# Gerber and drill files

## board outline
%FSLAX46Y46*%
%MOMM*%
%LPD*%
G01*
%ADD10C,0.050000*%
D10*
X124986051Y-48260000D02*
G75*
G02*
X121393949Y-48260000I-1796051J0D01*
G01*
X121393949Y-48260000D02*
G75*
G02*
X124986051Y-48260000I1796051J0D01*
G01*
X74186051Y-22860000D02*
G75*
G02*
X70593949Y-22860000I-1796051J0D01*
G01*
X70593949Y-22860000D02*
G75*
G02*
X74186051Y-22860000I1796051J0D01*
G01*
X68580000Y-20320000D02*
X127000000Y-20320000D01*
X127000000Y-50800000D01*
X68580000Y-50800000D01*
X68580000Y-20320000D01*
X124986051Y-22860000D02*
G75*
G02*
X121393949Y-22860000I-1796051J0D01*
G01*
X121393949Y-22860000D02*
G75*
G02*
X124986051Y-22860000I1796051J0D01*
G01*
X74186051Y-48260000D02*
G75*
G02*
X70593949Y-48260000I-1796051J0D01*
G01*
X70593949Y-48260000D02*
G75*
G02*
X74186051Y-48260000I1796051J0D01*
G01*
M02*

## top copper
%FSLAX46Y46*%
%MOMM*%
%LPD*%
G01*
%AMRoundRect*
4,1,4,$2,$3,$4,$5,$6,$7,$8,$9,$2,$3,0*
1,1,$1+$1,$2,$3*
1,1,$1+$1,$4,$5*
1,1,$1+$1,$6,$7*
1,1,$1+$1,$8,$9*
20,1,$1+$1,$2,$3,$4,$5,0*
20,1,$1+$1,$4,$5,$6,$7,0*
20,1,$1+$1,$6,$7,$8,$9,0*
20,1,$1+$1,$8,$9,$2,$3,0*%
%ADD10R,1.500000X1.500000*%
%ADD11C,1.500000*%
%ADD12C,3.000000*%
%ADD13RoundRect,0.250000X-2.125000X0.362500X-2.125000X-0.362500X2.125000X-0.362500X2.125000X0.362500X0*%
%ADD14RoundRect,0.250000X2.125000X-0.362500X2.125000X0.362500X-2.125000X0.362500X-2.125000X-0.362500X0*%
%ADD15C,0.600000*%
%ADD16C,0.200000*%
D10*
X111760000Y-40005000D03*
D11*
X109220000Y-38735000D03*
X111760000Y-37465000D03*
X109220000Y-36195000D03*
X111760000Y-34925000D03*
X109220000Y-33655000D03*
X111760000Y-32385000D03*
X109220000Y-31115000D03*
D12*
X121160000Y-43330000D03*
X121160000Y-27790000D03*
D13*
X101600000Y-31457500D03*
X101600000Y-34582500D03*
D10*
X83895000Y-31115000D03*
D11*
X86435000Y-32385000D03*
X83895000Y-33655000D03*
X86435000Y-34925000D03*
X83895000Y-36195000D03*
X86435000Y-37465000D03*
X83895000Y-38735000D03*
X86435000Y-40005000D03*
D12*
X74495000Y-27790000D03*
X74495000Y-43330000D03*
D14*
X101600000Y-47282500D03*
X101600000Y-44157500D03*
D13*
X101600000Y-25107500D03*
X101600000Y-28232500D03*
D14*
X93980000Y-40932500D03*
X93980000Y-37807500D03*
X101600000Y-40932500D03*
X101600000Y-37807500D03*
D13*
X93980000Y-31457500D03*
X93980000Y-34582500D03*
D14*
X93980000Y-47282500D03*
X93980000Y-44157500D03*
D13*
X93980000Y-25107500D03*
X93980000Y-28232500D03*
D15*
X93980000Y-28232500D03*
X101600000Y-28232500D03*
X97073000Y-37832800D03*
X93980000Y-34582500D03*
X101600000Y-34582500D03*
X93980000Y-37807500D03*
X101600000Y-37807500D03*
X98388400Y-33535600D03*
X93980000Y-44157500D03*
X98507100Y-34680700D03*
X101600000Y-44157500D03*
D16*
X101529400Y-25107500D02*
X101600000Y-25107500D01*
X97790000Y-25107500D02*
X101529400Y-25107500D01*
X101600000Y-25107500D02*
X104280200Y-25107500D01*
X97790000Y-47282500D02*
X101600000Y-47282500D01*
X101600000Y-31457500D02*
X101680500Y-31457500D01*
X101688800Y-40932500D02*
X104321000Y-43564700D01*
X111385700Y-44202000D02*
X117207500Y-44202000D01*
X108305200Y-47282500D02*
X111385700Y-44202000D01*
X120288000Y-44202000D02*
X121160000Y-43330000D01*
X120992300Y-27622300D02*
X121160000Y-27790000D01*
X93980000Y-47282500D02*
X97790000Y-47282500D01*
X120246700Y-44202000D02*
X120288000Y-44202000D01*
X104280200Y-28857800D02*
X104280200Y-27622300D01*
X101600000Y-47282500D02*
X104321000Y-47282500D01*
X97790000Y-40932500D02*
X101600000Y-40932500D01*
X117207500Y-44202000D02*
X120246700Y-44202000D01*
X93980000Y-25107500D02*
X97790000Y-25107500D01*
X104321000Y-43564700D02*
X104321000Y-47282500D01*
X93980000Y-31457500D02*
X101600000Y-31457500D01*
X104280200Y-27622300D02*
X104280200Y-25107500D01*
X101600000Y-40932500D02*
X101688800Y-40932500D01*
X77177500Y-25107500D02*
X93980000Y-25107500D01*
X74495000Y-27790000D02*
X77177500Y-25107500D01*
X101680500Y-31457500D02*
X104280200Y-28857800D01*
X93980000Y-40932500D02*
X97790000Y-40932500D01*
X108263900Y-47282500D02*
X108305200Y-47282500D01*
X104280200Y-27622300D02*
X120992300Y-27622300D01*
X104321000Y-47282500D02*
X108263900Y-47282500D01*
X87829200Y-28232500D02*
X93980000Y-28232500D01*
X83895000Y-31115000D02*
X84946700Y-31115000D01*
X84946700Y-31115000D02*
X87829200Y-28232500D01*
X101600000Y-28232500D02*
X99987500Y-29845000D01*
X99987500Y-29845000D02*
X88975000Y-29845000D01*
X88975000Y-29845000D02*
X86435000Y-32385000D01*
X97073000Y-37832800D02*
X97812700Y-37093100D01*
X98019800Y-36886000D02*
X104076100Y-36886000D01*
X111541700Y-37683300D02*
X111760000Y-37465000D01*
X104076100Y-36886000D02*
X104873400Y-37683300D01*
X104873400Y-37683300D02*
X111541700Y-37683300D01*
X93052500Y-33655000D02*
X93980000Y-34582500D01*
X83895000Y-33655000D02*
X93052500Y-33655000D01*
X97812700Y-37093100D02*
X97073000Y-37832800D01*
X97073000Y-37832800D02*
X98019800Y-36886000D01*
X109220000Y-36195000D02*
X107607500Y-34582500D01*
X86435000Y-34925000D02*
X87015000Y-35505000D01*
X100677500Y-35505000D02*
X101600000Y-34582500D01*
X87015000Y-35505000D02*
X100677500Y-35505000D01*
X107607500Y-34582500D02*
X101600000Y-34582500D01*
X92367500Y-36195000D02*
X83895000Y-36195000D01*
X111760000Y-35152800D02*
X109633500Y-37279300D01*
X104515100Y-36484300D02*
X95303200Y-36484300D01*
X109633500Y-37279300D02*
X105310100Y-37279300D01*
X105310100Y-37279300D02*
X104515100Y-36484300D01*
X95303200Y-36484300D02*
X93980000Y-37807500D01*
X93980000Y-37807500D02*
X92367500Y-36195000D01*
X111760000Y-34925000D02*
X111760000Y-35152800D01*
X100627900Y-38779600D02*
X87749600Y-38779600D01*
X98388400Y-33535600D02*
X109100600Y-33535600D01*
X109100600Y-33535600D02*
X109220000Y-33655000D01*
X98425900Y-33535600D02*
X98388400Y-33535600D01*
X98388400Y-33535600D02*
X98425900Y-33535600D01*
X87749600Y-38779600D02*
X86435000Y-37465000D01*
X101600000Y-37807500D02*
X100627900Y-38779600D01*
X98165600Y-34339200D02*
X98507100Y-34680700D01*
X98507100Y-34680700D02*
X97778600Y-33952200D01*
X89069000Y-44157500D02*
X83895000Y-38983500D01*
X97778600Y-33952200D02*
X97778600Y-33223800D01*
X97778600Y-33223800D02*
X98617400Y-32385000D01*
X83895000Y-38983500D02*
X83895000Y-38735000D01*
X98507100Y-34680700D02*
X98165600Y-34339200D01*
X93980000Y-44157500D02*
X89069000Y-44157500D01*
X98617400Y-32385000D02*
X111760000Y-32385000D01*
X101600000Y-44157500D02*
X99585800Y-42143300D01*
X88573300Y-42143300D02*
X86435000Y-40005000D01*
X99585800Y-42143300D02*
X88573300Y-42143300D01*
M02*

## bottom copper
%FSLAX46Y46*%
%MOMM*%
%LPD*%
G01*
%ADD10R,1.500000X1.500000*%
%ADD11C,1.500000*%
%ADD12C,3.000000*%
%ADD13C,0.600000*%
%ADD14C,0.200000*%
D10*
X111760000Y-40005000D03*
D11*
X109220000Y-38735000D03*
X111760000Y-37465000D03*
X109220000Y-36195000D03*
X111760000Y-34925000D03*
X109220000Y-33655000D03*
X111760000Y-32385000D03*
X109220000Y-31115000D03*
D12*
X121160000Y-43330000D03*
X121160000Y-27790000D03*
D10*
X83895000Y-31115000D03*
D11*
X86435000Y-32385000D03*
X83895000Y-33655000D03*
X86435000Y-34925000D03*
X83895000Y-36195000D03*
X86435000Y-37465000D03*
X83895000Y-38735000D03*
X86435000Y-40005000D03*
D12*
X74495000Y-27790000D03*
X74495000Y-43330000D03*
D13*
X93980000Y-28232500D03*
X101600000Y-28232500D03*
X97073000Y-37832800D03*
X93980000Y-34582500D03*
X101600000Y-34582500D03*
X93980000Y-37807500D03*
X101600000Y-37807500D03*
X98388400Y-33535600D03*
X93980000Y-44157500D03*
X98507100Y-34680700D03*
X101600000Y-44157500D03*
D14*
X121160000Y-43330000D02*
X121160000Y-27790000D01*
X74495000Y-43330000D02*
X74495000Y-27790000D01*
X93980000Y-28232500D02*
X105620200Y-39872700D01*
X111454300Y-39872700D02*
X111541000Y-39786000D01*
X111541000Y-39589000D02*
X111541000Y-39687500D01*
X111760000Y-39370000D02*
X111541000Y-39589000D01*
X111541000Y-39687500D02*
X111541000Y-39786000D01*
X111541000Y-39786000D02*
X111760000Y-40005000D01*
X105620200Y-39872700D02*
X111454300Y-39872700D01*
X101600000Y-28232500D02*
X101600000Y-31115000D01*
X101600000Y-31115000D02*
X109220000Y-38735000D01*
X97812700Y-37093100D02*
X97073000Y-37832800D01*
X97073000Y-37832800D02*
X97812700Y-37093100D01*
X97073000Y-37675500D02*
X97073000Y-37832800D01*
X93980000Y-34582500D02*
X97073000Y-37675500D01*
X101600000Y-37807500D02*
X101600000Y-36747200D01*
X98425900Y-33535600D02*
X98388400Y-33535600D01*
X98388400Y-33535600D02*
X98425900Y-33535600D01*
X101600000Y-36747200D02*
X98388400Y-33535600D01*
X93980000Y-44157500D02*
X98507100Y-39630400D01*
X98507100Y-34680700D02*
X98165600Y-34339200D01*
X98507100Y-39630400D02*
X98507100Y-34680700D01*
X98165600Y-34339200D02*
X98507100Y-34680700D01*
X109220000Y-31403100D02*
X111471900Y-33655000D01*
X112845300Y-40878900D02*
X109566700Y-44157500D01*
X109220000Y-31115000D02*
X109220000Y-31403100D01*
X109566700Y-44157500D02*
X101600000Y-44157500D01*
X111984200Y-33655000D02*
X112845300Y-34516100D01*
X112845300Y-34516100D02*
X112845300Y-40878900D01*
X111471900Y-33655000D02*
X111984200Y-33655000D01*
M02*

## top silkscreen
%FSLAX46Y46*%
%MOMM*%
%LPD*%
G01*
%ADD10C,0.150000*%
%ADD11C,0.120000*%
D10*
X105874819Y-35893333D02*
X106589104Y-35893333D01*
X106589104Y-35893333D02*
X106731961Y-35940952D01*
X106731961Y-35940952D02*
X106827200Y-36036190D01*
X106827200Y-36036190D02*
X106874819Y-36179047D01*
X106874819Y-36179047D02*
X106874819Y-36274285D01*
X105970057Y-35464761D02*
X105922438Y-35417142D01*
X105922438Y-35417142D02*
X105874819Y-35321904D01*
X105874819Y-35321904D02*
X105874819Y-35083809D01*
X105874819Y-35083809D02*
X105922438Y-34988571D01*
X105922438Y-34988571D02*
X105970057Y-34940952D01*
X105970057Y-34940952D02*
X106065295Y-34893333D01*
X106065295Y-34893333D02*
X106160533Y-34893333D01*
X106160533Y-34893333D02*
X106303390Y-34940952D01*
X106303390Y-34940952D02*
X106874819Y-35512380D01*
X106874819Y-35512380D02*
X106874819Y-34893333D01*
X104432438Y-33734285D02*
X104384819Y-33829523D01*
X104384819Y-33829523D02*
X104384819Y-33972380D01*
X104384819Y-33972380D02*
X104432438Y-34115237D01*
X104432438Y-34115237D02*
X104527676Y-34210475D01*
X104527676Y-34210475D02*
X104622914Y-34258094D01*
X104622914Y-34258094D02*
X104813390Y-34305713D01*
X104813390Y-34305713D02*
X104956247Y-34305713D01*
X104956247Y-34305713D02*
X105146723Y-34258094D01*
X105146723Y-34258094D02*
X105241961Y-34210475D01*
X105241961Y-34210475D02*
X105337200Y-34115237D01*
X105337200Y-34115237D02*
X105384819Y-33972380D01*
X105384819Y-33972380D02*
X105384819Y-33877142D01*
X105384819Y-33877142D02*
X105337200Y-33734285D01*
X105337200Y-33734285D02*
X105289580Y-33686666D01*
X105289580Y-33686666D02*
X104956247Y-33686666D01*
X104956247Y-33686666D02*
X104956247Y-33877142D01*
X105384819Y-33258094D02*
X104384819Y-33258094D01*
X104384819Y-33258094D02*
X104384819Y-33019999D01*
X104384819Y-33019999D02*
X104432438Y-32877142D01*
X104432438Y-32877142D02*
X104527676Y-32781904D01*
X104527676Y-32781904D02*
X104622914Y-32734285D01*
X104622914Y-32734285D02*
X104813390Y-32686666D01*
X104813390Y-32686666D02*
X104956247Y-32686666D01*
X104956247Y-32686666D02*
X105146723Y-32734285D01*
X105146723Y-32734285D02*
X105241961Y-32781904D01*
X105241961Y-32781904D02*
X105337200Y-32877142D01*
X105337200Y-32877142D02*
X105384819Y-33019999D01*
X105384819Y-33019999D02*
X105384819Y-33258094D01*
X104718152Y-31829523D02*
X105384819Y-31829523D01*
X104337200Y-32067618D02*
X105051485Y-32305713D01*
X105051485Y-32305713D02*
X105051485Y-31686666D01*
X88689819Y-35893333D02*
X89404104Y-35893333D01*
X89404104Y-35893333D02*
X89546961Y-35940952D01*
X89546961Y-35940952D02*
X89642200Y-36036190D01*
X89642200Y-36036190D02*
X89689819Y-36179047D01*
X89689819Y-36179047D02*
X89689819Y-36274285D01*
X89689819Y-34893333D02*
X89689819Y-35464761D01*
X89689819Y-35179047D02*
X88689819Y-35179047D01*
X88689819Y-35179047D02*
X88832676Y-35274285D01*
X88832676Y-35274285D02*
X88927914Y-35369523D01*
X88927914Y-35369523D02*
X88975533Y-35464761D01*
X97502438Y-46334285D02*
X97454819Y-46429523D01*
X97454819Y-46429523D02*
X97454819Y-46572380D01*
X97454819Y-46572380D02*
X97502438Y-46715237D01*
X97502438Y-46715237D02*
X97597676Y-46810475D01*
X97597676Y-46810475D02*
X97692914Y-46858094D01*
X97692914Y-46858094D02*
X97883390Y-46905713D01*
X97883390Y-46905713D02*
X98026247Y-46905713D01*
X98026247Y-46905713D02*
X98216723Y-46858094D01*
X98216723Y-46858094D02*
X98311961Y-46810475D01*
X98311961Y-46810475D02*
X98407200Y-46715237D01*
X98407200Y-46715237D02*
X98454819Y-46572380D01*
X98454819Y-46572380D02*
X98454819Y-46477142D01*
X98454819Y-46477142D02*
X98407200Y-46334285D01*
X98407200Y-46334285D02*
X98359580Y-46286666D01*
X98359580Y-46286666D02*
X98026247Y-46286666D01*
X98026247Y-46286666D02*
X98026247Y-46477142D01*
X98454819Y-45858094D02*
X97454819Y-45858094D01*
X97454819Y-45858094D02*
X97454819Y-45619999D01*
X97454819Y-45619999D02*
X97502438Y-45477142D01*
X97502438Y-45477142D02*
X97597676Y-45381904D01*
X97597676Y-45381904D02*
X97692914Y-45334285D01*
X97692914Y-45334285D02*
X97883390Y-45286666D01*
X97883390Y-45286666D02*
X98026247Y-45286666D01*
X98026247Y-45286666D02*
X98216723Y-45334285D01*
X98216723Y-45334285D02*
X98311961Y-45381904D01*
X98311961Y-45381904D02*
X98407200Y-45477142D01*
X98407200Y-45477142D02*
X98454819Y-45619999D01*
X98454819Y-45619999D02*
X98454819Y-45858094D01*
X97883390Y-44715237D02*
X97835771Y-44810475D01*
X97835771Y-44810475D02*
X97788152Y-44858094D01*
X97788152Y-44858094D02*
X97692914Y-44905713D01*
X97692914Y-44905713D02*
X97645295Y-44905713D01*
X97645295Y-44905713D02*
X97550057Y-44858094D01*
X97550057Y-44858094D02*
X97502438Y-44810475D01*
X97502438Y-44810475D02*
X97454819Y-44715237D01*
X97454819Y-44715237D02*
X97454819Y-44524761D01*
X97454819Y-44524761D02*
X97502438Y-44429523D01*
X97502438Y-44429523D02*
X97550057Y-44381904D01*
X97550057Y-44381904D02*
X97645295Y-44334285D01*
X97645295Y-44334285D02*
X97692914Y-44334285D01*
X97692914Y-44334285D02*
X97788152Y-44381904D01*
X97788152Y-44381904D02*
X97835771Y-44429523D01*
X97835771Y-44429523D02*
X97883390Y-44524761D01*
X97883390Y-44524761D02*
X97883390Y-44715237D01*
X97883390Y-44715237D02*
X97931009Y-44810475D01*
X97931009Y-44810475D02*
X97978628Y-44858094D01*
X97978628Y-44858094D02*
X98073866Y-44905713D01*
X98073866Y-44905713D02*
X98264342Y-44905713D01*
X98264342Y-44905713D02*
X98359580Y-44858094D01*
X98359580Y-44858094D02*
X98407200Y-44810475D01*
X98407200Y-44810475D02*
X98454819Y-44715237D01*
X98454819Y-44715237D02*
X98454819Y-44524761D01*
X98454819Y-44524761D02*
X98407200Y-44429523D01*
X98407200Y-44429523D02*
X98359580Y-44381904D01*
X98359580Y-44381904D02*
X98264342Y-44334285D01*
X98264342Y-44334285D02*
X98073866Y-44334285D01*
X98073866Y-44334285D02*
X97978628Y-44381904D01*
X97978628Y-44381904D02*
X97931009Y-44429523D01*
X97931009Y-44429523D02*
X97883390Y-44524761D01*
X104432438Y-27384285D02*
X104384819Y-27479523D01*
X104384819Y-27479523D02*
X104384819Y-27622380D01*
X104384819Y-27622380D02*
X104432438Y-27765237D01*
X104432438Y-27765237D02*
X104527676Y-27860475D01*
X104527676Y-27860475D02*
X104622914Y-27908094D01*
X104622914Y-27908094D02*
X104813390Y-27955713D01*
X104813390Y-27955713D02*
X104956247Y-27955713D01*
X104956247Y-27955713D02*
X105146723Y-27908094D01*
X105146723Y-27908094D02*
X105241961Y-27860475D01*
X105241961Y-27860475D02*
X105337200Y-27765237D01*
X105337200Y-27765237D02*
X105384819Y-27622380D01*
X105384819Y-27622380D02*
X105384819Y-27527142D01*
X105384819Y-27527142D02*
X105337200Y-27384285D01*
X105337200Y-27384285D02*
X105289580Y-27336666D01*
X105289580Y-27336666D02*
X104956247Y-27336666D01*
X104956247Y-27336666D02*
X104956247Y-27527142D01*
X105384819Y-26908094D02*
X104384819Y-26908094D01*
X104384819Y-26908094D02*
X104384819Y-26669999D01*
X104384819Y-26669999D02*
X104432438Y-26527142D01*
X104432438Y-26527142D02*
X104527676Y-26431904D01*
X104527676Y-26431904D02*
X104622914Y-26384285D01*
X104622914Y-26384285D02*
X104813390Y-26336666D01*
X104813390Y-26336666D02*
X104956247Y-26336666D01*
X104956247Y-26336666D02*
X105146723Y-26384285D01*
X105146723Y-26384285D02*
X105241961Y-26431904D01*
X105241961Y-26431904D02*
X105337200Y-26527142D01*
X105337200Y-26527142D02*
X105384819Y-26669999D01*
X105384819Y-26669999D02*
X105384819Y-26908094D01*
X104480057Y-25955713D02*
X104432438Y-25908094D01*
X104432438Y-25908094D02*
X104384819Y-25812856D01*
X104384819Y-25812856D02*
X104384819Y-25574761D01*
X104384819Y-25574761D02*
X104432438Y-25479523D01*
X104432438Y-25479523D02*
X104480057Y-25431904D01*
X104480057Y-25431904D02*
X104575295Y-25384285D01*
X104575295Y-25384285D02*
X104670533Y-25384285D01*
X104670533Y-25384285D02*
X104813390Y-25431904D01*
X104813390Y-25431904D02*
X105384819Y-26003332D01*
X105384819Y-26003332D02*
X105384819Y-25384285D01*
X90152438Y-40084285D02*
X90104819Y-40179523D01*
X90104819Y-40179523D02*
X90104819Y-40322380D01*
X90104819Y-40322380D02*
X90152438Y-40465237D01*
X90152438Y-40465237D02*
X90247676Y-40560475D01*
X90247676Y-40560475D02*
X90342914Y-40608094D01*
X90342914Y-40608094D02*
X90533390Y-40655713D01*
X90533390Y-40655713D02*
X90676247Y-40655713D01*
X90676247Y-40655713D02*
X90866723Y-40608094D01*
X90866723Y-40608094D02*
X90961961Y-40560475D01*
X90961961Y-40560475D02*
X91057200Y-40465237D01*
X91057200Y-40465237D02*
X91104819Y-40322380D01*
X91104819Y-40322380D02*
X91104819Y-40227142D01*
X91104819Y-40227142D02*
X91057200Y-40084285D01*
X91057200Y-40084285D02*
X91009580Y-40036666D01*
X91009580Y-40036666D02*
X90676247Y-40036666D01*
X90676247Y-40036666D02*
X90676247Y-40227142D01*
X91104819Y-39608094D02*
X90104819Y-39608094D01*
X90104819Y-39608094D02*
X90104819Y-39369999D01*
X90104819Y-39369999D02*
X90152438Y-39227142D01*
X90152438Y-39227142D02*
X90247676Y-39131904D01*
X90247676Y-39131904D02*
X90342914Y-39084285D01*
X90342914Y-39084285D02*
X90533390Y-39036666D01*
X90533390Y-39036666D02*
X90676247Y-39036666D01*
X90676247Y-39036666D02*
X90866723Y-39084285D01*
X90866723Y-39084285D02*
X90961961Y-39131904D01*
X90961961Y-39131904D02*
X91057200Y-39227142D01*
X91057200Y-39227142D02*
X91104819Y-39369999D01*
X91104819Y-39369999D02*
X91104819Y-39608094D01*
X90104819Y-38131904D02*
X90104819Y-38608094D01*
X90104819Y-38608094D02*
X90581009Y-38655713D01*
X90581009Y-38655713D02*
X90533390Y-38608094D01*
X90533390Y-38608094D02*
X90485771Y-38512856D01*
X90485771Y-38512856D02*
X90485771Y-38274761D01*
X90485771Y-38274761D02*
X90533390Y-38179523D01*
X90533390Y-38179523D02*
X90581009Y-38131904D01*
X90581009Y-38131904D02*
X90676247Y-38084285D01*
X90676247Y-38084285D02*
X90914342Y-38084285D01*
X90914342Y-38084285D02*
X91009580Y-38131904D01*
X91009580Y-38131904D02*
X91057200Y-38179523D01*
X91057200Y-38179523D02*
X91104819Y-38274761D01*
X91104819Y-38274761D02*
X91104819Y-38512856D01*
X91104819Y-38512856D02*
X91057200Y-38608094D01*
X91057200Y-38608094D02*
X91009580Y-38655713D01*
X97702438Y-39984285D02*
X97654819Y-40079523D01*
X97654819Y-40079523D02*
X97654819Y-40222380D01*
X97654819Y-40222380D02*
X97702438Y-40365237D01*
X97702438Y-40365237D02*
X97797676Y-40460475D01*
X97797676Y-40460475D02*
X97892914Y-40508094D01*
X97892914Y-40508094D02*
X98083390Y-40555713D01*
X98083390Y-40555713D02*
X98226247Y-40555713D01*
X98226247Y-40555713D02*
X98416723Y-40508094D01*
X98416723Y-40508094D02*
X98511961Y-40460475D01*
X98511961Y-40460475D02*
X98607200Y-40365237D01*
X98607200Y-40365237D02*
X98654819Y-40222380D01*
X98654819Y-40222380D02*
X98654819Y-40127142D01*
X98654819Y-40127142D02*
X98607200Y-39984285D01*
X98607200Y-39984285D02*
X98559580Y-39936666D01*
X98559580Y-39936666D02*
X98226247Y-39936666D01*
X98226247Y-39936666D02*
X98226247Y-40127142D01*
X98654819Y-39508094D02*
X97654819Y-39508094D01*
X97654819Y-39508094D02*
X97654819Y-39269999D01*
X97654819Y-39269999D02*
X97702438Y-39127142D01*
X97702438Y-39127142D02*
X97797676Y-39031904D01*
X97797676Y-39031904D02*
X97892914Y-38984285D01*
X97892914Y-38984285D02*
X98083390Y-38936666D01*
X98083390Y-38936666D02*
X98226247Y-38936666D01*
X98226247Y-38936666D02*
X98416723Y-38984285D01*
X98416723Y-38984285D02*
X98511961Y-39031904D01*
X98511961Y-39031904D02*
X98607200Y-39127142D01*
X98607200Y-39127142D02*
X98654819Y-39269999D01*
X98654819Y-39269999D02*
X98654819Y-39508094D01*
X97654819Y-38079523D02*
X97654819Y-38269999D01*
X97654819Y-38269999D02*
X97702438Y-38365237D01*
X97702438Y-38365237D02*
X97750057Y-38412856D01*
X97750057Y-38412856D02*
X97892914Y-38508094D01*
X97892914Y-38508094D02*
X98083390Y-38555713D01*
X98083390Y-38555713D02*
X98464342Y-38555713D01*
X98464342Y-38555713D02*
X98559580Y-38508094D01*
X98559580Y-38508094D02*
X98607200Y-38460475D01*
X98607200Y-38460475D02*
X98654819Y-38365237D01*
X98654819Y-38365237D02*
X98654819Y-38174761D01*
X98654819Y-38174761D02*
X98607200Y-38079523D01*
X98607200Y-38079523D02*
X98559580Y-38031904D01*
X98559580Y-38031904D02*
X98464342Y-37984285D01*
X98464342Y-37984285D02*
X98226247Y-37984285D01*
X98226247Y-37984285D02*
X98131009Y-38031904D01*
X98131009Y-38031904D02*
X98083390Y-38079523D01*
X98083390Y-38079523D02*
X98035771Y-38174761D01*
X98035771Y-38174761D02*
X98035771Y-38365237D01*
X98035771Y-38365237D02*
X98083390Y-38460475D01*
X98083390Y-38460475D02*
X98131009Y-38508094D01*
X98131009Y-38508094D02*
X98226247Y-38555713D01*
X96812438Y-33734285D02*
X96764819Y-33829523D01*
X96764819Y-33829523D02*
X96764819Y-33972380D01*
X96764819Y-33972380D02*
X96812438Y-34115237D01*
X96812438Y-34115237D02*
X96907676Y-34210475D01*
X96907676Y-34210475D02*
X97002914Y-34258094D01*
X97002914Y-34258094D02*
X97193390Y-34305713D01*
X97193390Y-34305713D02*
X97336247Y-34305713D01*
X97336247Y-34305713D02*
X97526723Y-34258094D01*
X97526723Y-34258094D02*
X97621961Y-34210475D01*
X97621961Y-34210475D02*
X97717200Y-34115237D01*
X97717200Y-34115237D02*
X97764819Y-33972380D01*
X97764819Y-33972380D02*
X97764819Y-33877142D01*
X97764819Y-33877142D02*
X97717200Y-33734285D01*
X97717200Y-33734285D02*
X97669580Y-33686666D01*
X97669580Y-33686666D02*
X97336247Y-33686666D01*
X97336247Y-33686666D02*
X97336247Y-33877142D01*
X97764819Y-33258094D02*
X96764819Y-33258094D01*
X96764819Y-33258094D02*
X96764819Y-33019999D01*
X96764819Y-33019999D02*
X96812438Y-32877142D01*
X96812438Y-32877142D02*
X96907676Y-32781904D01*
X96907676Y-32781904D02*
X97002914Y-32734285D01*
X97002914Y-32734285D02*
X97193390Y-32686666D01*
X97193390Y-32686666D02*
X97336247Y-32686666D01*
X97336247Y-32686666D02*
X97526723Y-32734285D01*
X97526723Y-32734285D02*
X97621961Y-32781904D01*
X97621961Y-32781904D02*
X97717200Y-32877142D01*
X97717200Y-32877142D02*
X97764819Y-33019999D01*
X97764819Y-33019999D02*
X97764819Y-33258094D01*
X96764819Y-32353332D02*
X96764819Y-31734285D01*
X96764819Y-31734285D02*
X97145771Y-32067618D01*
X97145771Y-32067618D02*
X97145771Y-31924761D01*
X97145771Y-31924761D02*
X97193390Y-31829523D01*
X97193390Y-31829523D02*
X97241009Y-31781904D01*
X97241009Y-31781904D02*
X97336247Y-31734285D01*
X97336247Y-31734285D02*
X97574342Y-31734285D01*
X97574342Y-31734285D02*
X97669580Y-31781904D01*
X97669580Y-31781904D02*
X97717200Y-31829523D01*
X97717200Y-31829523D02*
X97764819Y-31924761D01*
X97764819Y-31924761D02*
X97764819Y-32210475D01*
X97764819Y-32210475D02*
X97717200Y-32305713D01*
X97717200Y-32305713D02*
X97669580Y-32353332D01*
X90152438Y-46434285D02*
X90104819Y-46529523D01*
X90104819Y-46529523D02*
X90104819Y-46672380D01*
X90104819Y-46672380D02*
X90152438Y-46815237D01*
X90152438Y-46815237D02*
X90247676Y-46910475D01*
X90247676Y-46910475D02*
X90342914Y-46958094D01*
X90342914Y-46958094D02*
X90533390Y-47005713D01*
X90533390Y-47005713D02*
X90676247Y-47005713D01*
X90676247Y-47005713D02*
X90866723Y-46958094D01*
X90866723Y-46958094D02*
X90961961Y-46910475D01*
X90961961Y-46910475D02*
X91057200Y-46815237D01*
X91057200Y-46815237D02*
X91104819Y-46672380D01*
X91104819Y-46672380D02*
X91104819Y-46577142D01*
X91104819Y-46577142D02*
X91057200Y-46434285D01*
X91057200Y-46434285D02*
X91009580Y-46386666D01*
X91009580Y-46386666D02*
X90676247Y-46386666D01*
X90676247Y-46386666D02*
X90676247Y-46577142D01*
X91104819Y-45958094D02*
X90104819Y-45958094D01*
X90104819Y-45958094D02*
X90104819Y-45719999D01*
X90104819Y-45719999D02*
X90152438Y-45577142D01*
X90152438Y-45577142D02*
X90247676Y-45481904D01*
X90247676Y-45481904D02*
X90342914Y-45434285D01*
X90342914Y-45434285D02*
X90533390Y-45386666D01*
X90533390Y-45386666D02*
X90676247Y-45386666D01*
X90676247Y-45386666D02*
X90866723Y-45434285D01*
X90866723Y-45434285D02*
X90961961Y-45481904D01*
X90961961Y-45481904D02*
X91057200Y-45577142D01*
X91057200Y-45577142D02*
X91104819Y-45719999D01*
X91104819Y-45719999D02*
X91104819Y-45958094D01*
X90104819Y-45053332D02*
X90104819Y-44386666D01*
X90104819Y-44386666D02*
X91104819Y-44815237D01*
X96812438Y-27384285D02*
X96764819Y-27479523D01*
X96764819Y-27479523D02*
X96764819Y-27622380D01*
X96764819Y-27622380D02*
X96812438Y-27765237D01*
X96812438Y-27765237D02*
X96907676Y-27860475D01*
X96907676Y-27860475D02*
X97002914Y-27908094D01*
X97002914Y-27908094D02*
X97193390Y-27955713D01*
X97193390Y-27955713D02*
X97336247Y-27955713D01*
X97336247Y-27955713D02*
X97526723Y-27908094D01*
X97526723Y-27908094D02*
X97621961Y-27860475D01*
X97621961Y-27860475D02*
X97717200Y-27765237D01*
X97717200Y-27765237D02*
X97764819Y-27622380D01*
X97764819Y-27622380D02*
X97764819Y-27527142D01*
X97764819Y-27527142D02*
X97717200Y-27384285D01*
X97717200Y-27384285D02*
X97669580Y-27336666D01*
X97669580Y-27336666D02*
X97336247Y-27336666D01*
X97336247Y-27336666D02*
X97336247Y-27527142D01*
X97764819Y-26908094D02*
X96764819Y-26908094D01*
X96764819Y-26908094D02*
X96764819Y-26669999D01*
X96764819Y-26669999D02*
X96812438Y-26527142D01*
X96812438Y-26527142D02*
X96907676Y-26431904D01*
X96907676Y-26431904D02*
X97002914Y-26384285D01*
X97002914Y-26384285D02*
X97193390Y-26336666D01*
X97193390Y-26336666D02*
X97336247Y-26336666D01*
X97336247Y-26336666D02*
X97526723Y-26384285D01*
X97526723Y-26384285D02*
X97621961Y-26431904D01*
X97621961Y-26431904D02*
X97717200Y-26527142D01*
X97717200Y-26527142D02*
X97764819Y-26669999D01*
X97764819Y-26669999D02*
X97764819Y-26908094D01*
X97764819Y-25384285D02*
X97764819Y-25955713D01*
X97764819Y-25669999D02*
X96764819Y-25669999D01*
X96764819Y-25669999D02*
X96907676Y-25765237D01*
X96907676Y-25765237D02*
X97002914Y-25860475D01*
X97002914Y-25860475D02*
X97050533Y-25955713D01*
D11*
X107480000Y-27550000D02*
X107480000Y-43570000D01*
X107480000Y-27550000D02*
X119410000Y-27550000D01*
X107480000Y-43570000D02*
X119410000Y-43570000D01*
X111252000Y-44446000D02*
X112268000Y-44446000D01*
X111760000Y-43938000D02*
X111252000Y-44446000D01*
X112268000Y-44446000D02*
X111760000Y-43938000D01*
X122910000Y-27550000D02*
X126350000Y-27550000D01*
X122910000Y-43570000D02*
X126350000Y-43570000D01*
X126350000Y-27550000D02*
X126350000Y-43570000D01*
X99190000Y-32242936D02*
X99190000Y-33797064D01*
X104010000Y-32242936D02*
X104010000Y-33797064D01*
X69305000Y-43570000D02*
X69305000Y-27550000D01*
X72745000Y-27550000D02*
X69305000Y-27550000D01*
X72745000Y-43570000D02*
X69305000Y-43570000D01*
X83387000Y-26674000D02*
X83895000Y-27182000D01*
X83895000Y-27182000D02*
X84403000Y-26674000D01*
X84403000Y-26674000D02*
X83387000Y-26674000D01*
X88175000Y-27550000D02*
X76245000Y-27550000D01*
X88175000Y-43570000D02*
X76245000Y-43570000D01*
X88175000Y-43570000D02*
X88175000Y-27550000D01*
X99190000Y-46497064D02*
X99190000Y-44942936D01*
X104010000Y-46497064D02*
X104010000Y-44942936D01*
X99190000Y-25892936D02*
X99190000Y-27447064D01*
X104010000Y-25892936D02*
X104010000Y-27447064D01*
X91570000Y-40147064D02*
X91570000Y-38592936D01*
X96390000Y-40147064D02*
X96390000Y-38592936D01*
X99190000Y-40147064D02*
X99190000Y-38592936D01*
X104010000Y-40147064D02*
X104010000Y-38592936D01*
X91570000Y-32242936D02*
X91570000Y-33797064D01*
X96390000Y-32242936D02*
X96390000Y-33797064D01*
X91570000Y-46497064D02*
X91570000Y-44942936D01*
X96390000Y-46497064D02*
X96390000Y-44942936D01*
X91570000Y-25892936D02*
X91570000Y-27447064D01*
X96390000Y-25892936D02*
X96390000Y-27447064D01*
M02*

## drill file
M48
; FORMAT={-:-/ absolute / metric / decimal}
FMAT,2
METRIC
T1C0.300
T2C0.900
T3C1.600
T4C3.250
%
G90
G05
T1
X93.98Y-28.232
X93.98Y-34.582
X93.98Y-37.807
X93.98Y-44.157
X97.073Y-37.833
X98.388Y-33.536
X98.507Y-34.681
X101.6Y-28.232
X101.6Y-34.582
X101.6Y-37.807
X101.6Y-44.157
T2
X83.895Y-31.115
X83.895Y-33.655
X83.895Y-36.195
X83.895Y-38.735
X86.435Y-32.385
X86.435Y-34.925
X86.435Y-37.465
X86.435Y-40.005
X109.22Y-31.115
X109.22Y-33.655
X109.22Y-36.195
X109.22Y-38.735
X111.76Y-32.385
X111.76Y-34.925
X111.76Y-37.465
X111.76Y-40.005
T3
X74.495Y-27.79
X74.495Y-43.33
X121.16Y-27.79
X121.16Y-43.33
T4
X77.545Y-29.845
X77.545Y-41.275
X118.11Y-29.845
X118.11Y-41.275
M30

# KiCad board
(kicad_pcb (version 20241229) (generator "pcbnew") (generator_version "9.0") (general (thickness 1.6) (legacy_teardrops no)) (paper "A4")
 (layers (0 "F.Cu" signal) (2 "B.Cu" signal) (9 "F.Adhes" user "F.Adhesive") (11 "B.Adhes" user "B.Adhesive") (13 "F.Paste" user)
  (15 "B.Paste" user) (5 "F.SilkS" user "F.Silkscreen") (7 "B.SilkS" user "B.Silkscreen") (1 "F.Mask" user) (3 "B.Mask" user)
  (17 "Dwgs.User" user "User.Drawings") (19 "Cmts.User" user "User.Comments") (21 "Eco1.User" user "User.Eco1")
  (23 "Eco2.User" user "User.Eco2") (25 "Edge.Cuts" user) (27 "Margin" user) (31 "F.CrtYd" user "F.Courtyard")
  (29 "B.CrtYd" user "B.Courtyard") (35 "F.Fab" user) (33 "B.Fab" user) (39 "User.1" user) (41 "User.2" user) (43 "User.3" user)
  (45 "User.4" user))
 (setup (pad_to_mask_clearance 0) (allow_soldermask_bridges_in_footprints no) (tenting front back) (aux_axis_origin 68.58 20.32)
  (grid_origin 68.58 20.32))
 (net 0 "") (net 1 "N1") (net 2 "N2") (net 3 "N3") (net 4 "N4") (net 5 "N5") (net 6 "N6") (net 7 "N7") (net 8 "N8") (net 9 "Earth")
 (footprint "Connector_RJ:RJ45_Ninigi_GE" (layer "F.Cu") (at 111.76 40.005 90)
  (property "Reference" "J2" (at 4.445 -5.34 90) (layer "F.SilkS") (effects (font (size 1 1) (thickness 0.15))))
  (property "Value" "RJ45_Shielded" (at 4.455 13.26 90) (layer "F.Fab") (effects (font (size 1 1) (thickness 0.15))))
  (fp_line (start 12.455 -4.28) (end -3.565 -4.28) (stroke (width 0.12) (type solid)) (layer "F.SilkS"))
  (fp_line (start 12.455 -4.28) (end 12.455 7.65) (stroke (width 0.12) (type solid)) (layer "F.SilkS"))
  (fp_line (start -3.565 -4.28) (end -3.565 7.65) (stroke (width 0.12) (type solid)) (layer "F.SilkS"))
  (fp_line (start -4.441 -0.508) (end -4.441 0.508) (stroke (width 0.12) (type solid)) (layer "F.SilkS"))
  (fp_line (start -3.933 0) (end -4.441 -0.508) (stroke (width 0.12) (type solid)) (layer "F.SilkS"))
  (fp_line (start -4.441 0.508) (end -3.933 0) (stroke (width 0.12) (type solid)) (layer "F.SilkS"))
  (fp_line (start 12.455 11.15) (end 12.455 14.59) (stroke (width 0.12) (type solid)) (layer "F.SilkS"))
  (fp_line (start -3.565 11.15) (end -3.565 14.59) (stroke (width 0.12) (type solid)) (layer "F.SilkS"))
  (fp_line (start 12.455 14.59) (end -3.565 14.59) (stroke (width 0.12) (type solid)) (layer "F.SilkS"))
  (pad "" np_thru_hole circle (at -1.27 6.35 90) (size 3.25 3.25) (drill 3.25) (layers "*.Cu" "*.Mask"))
  (pad "" np_thru_hole circle (at 10.16 6.35 270) (size 3.25 3.25) (drill 3.25) (layers "*.Cu" "*.Mask"))
  (pad "1" thru_hole rect (at 0 0 270) (size 1.5 1.5) (drill 0.9) (layers "*.Cu" "*.Mask") (remove_unused_layers no) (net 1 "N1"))
  (pad "2" thru_hole circle (at 1.27 -2.54 270) (size 1.5 1.5) (drill 0.9) (layers "*.Cu" "*.Mask") (remove_unused_layers no) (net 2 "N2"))
  (pad "3" thru_hole circle (at 2.54 0 270) (size 1.5 1.5) (drill 0.9) (layers "*.Cu" "*.Mask") (remove_unused_layers no) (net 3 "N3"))
  (pad "4" thru_hole circle (at 3.81 -2.54 270) (size 1.5 1.5) (drill 0.9) (layers "*.Cu" "*.Mask") (remove_unused_layers no) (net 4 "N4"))
  (pad "5" thru_hole circle (at 5.08 0 270) (size 1.5 1.5) (drill 0.9) (layers "*.Cu" "*.Mask") (remove_unused_layers no) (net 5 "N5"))
  (pad "6" thru_hole circle (at 6.35 -2.54 270) (size 1.5 1.5) (drill 0.9) (layers "*.Cu" "*.Mask") (remove_unused_layers no) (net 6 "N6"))
  (pad "7" thru_hole circle (at 7.62 0 270) (size 1.5 1.5) (drill 0.9) (layers "*.Cu" "*.Mask") (remove_unused_layers no) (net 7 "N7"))
  (pad "8" thru_hole circle (at 8.89 -2.54 270) (size 1.5 1.5) (drill 0.9) (layers "*.Cu" "*.Mask") (remove_unused_layers no) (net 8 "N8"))
  (pad "SH" thru_hole circle (at -3.325 9.4 90) (size 3 3) (drill 1.6) (layers "*.Cu" "*.Mask") (remove_unused_layers no) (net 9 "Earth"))
  (pad "SH" thru_hole circle (at 12.215 9.4 270) (size 3 3) (drill 1.6) (layers "*.Cu" "*.Mask") (remove_unused_layers no) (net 9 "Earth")))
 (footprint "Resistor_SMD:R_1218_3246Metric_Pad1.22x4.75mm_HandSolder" (layer "F.Cu") (at 101.6 33.02 -90)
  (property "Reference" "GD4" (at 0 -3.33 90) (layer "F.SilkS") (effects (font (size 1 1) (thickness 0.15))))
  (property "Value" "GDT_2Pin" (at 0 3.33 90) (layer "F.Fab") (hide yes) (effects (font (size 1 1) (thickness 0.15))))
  (fp_line (start -0.777064 2.41) (end 0.777064 2.41) (stroke (width 0.12) (type solid)) (layer "F.SilkS"))
  (fp_line (start -0.777064 -2.41) (end 0.777064 -2.41) (stroke (width 0.12) (type solid)) (layer "F.SilkS"))
  (pad "1" smd roundrect (at -1.5625 0 270) (size 1.225 4.75) (layers "F.Cu" "F.Mask" "F.Paste") (roundrect_rratio 0.204082) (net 9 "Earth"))
  (pad "2" smd roundrect (at 1.5625 0 270) (size 1.225 4.75) (layers "F.Cu" "F.Mask" "F.Paste") (roundrect_rratio 0.204082) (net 4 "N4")))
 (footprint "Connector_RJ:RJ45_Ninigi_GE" (layer "F.Cu") (at 83.895 31.115 -90)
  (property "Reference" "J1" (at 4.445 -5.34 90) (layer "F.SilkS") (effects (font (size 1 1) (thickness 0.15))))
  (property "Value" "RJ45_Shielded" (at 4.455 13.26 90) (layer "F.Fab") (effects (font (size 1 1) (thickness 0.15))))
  (fp_line (start 12.455 14.59) (end -3.565 14.59) (stroke (width 0.12) (type solid)) (layer "F.SilkS"))
  (fp_line (start -3.565 11.15) (end -3.565 14.59) (stroke (width 0.12) (type solid)) (layer "F.SilkS"))
  (fp_line (start 12.455 11.15) (end 12.455 14.59) (stroke (width 0.12) (type solid)) (layer "F.SilkS"))
  (fp_line (start -4.441 0.508) (end -3.933 0) (stroke (width 0.12) (type solid)) (layer "F.SilkS"))
  (fp_line (start -3.933 0) (end -4.441 -0.508) (stroke (width 0.12) (type solid)) (layer "F.SilkS"))
  (fp_line (start -4.441 -0.508) (end -4.441 0.508) (stroke (width 0.12) (type solid)) (layer "F.SilkS"))
  (fp_line (start -3.565 -4.28) (end -3.565 7.65) (stroke (width 0.12) (type solid)) (layer "F.SilkS"))
  (fp_line (start 12.455 -4.28) (end 12.455 7.65) (stroke (width 0.12) (type solid)) (layer "F.SilkS"))
  (fp_line (start 12.455 -4.28) (end -3.565 -4.28) (stroke (width 0.12) (type solid)) (layer "F.SilkS"))
  (pad "" np_thru_hole circle (at -1.27 6.35 270) (size 3.25 3.25) (drill 3.25) (layers "*.Cu" "*.Mask"))
  (pad "" np_thru_hole circle (at 10.16 6.35 90) (size 3.25 3.25) (drill 3.25) (layers "*.Cu" "*.Mask"))
  (pad "1" thru_hole rect (at 0 0 90) (size 1.5 1.5) (drill 0.9) (layers "*.Cu" "*.Mask") (remove_unused_layers no) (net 1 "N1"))
  (pad "2" thru_hole circle (at 1.27 -2.54 90) (size 1.5 1.5) (drill 0.9) (layers "*.Cu" "*.Mask") (remove_unused_layers no) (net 2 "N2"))
  (pad "3" thru_hole circle (at 2.54 0 90) (size 1.5 1.5) (drill 0.9) (layers "*.Cu" "*.Mask") (remove_unused_layers no) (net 3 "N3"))
  (pad "4" thru_hole circle (at 3.81 -2.54 90) (size 1.5 1.5) (drill 0.9) (layers "*.Cu" "*.Mask") (remove_unused_layers no) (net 4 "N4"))
  (pad "5" thru_hole circle (at 5.08 0 90) (size 1.5 1.5) (drill 0.9) (layers "*.Cu" "*.Mask") (remove_unused_layers no) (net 5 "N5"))
  (pad "6" thru_hole circle (at 6.35 -2.54 90) (size 1.5 1.5) (drill 0.9) (layers "*.Cu" "*.Mask") (remove_unused_layers no) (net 6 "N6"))
  (pad "7" thru_hole circle (at 7.62 0 90) (size 1.5 1.5) (drill 0.9) (layers "*.Cu" "*.Mask") (remove_unused_layers no) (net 7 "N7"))
  (pad "8" thru_hole circle (at 8.89 -2.54 90) (size 1.5 1.5) (drill 0.9) (layers "*.Cu" "*.Mask") (remove_unused_layers no) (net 8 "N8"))
  (pad "SH" thru_hole circle (at -3.325 9.4 270) (size 3 3) (drill 1.6) (layers "*.Cu" "*.Mask") (remove_unused_layers no) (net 9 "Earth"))
  (pad "SH" thru_hole circle (at 12.215 9.4 90) (size 3 3) (drill 1.6) (layers "*.Cu" "*.Mask") (remove_unused_layers no) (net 9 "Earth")))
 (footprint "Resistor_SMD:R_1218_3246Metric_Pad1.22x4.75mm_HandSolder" (layer "F.Cu") (at 101.6 45.72 90)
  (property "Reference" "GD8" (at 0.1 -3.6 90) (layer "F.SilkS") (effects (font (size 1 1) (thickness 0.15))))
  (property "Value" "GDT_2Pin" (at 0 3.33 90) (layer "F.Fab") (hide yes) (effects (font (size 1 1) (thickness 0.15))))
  (fp_line (start -0.777064 -2.41) (end 0.777064 -2.41) (stroke (width 0.12) (type solid)) (layer "F.SilkS"))
  (fp_line (start -0.777064 2.41) (end 0.777064 2.41) (stroke (width 0.12) (type solid)) (layer "F.SilkS"))
  (pad "1" smd roundrect (at -1.5625 0 90) (size 1.225 4.75) (layers "F.Cu" "F.Mask" "F.Paste") (roundrect_rratio 0.204082) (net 9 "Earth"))
  (pad "2" smd roundrect (at 1.5625 0 90) (size 1.225 4.75) (layers "F.Cu" "F.Mask" "F.Paste") (roundrect_rratio 0.204082) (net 8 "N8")))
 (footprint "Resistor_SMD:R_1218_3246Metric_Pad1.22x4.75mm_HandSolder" (layer "F.Cu") (at 101.6 26.67 -90)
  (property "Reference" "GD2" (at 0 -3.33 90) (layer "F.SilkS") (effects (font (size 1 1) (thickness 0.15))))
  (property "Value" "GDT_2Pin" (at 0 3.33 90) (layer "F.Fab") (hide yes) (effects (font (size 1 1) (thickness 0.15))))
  (fp_line (start -0.777064 2.41) (end 0.777064 2.41) (stroke (width 0.12) (type solid)) (layer "F.SilkS"))
  (fp_line (start -0.777064 -2.41) (end 0.777064 -2.41) (stroke (width 0.12) (type solid)) (layer "F.SilkS"))
  (pad "1" smd roundrect (at -1.5625 0 270) (size 1.225 4.75) (layers "F.Cu" "F.Mask" "F.Paste") (roundrect_rratio 0.204082) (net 9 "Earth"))
  (pad "2" smd roundrect (at 1.5625 0 270) (size 1.225 4.75) (layers "F.Cu" "F.Mask" "F.Paste") (roundrect_rratio 0.204082) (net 2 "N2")))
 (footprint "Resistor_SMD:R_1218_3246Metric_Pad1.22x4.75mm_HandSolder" (layer "F.Cu") (at 93.98 39.37 90)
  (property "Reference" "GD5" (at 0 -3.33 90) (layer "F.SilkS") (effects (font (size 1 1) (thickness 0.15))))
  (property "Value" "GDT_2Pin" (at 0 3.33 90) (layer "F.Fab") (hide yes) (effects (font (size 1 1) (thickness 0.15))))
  (fp_line (start -0.777064 -2.41) (end 0.777064 -2.41) (stroke (width 0.12) (type solid)) (layer "F.SilkS"))
  (fp_line (start -0.777064 2.41) (end 0.777064 2.41) (stroke (width 0.12) (type solid)) (layer "F.SilkS"))
  (pad "1" smd roundrect (at -1.5625 0 90) (size 1.225 4.75) (layers "F.Cu" "F.Mask" "F.Paste") (roundrect_rratio 0.204082) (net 9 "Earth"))
  (pad "2" smd roundrect (at 1.5625 0 90) (size 1.225 4.75) (layers "F.Cu" "F.Mask" "F.Paste") (roundrect_rratio 0.204082) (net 5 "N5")))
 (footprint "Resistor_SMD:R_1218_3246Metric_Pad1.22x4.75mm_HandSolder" (layer "F.Cu") (at 101.6 39.37 90)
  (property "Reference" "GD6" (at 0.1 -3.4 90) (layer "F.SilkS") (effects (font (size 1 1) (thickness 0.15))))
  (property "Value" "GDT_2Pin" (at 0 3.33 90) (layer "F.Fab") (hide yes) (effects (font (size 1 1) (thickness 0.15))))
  (fp_line (start -0.777064 -2.41) (end 0.777064 -2.41) (stroke (width 0.12) (type solid)) (layer "F.SilkS"))
  (fp_line (start -0.777064 2.41) (end 0.777064 2.41) (stroke (width 0.12) (type solid)) (layer "F.SilkS"))
  (pad "1" smd roundrect (at -1.5625 0 90) (size 1.225 4.75) (layers "F.Cu" "F.Mask" "F.Paste") (roundrect_rratio 0.204082) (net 9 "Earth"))
  (pad "2" smd roundrect (at 1.5625 0 90) (size 1.225 4.75) (layers "F.Cu" "F.Mask" "F.Paste") (roundrect_rratio 0.204082) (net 6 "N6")))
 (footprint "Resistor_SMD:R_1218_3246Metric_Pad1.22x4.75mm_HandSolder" (layer "F.Cu") (at 93.98 33.02 -90)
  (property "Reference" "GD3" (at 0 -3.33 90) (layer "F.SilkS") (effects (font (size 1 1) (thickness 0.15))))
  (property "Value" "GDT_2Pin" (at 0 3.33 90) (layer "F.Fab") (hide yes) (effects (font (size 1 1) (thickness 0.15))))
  (fp_line (start -0.777064 2.41) (end 0.777064 2.41) (stroke (width 0.12) (type solid)) (layer "F.SilkS"))
  (fp_line (start -0.777064 -2.41) (end 0.777064 -2.41) (stroke (width 0.12) (type solid)) (layer "F.SilkS"))
  (pad "1" smd roundrect (at -1.5625 0 270) (size 1.225 4.75) (layers "F.Cu" "F.Mask" "F.Paste") (roundrect_rratio 0.204082) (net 9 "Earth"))
  (pad "2" smd roundrect (at 1.5625 0 270) (size 1.225 4.75) (layers "F.Cu" "F.Mask" "F.Paste") (roundrect_rratio 0.204082) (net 3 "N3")))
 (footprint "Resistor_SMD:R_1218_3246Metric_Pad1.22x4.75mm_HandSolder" (layer "F.Cu") (at 93.98 45.72 90)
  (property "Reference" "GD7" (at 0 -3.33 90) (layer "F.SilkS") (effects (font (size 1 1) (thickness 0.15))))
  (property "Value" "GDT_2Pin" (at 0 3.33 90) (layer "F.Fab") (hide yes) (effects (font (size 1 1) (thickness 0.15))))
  (fp_line (start -0.777064 -2.41) (end 0.777064 -2.41) (stroke (width 0.12) (type solid)) (layer "F.SilkS"))
  (fp_line (start -0.777064 2.41) (end 0.777064 2.41) (stroke (width 0.12) (type solid)) (layer "F.SilkS"))
  (pad "1" smd roundrect (at -1.5625 0 90) (size 1.225 4.75) (layers "F.Cu" "F.Mask" "F.Paste") (roundrect_rratio 0.204082) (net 9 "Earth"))
  (pad "2" smd roundrect (at 1.5625 0 90) (size 1.225 4.75) (layers "F.Cu" "F.Mask" "F.Paste") (roundrect_rratio 0.204082) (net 7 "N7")))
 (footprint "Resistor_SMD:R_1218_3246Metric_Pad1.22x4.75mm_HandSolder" (layer "F.Cu") (at 93.98 26.67 -90)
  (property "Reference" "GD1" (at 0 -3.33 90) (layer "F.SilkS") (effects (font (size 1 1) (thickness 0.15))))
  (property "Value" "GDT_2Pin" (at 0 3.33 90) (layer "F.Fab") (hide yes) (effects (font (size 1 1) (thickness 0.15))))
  (fp_line (start -0.777064 2.41) (end 0.777064 2.41) (stroke (width 0.12) (type solid)) (layer "F.SilkS"))
  (fp_line (start -0.777064 -2.41) (end 0.777064 -2.41) (stroke (width 0.12) (type solid)) (layer "F.SilkS"))
  (pad "1" smd roundrect (at -1.5625 0 270) (size 1.225 4.75) (layers "F.Cu" "F.Mask" "F.Paste") (roundrect_rratio 0.204082) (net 9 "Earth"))
  (pad "2" smd roundrect (at 1.5625 0 270) (size 1.225 4.75) (layers "F.Cu" "F.Mask" "F.Paste") (roundrect_rratio 0.204082) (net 1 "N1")))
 (gr_circle (center 123.19 48.26) (end 121.92 46.99) (stroke (width 0.05) (type default)) (fill no) (layer "Edge.Cuts"))
 (gr_circle (center 72.39 22.86) (end 73.66 24.13) (stroke (width 0.05) (type default)) (fill no) (layer "Edge.Cuts"))
 (gr_rect (start 68.58 20.32) (end 127 50.8) (stroke (width 0.05) (type default)) (fill no) (layer "Edge.Cuts"))
 (gr_circle (center 123.19 22.86) (end 124.46 24.13) (stroke (width 0.05) (type default)) (fill no) (layer "Edge.Cuts"))
 (gr_circle (center 72.39 48.26) (end 71.12 46.99) (stroke (width 0.05) (type default)) (fill no) (layer "Edge.Cuts"))
 (segment (start 101.5294 25.1075) (end 101.6 25.1075) (width 0.2) (layer "F.Cu") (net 9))
 (segment (start 97.79 25.1075) (end 101.5294 25.1075) (width 0.2) (layer "F.Cu") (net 9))
 (segment (start 101.6 25.1075) (end 104.2802 25.1075) (width 0.2) (layer "F.Cu") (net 9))
 (segment (start 97.79 47.2825) (end 101.6 47.2825) (width 0.2) (layer "F.Cu") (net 9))
 (segment (start 101.6 31.4575) (end 101.6805 31.4575) (width 0.2) (layer "F.Cu") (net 9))
 (segment (start 101.6888 40.9325) (end 104.321 43.5647) (width 0.2) (layer "F.Cu") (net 9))
 (segment (start 111.3857 44.202) (end 117.2075 44.202) (width 0.2) (layer "F.Cu") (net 9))
 (segment (start 108.3052 47.2825) (end 111.3857 44.202) (width 0.2) (layer "F.Cu") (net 9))
 (segment (start 120.288 44.202) (end 121.16 43.33) (width 0.2) (layer "F.Cu") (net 9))
 (segment (start 120.9923 27.6223) (end 121.16 27.79) (width 0.2) (layer "F.Cu") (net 9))
 (segment (start 93.98 47.2825) (end 97.79 47.2825) (width 0.2) (layer "F.Cu") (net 9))
 (segment (start 120.2467 44.202) (end 120.288 44.202) (width 0.2) (layer "F.Cu") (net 9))
 (segment (start 104.2802 28.8578) (end 104.2802 27.6223) (width 0.2) (layer "F.Cu") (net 9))
 (segment (start 101.6 47.2825) (end 104.321 47.2825) (width 0.2) (layer "F.Cu") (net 9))
 (segment (start 97.79 40.9325) (end 101.6 40.9325) (width 0.2) (layer "F.Cu") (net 9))
 (segment (start 117.2075 44.202) (end 120.2467 44.202) (width 0.2) (layer "F.Cu") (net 9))
 (segment (start 93.98 25.1075) (end 97.79 25.1075) (width 0.2) (layer "F.Cu") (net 9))
 (segment (start 104.321 43.5647) (end 104.321 47.2825) (width 0.2) (layer "F.Cu") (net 9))
 (segment (start 93.98 31.4575) (end 101.6 31.4575) (width 0.2) (layer "F.Cu") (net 9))
 (segment (start 104.2802 27.6223) (end 104.2802 25.1075) (width 0.2) (layer "F.Cu") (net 9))
 (segment (start 101.6 40.9325) (end 101.6888 40.9325) (width 0.2) (layer "F.Cu") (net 9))
 (segment (start 77.1775 25.1075) (end 93.98 25.1075) (width 0.2) (layer "F.Cu") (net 9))
 (segment (start 74.495 27.79) (end 77.1775 25.1075) (width 0.2) (layer "F.Cu") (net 9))
 (segment (start 101.6805 31.4575) (end 104.2802 28.8578) (width 0.2) (layer "F.Cu") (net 9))
 (segment (start 93.98 40.9325) (end 97.79 40.9325) (width 0.2) (layer "F.Cu") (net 9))
 (segment (start 108.2639 47.2825) (end 108.3052 47.2825) (width 0.2) (layer "F.Cu") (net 9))
 (segment (start 104.2802 27.6223) (end 120.9923 27.6223) (width 0.2) (layer "F.Cu") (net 9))
 (segment (start 104.321 47.2825) (end 108.2639 47.2825) (width 0.2) (layer "F.Cu") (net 9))
 (segment (start 121.16 43.33) (end 121.16 27.79) (width 0.2) (layer "B.Cu") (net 9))
 (segment (start 74.495 43.33) (end 74.495 27.79) (width 0.2) (layer "B.Cu") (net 9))
 (segment (start 87.8292 28.2325) (end 93.98 28.2325) (width 0.2) (layer "F.Cu") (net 1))
 (segment (start 83.895 31.115) (end 84.9467 31.115) (width 0.2) (layer "F.Cu") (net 1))
 (segment (start 84.9467 31.115) (end 87.8292 28.2325) (width 0.2) (layer "F.Cu") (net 1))
 (via (at 93.98 28.2325) (size 0.6) (drill 0.3) (layers "F.Cu" "B.Cu") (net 1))
 (segment (start 93.98 28.2325) (end 105.6202 39.8727) (width 0.2) (layer "B.Cu") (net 1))
 (segment (start 111.4543 39.8727) (end 111.541 39.786) (width 0.2) (layer "B.Cu") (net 1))
 (segment (start 111.541 39.589) (end 111.541 39.6875) (width 0.2) (layer "B.Cu") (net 1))
 (segment (start 111.76 39.37) (end 111.541 39.589) (width 0.2) (layer "B.Cu") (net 1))
 (segment (start 111.541 39.6875) (end 111.541 39.786) (width 0.2) (layer "B.Cu") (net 1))
 (segment (start 111.541 39.786) (end 111.76 40.005) (width 0.2) (layer "B.Cu") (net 1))
 (segment (start 105.6202 39.8727) (end 111.4543 39.8727) (width 0.2) (layer "B.Cu") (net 1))
 (segment (start 101.6 28.2325) (end 99.9875 29.845) (width 0.2) (layer "F.Cu") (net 2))
 (segment (start 99.9875 29.845) (end 88.975 29.845) (width 0.2) (layer "F.Cu") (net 2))
 (segment (start 88.975 29.845) (end 86.435 32.385) (width 0.2) (layer "F.Cu") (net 2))
 (via (at 101.6 28.2325) (size 0.6) (drill 0.3) (layers "F.Cu" "B.Cu") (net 2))
 (segment (start 101.6 28.2325) (end 101.6 31.115) (width 0.2) (layer "B.Cu") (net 2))
 (segment (start 101.6 31.115) (end 109.22 38.735) (width 0.2) (layer "B.Cu") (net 2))
 (segment (start 97.073 37.8328) (end 97.8127 37.0931) (width 0.2) (layer "F.Cu") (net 3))
 (segment (start 98.0198 36.886) (end 104.0761 36.886) (width 0.2) (layer "F.Cu") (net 3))
 (segment (start 111.5417 37.6833) (end 111.76 37.465) (width 0.2) (layer "F.Cu") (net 3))
 (segment (start 104.0761 36.886) (end 104.8734 37.6833) (width 0.2) (layer "F.Cu") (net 3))
 (segment (start 104.8734 37.6833) (end 111.5417 37.6833) (width 0.2) (layer "F.Cu") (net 3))
 (segment (start 93.0525 33.655) (end 93.98 34.5825) (width 0.2) (layer "F.Cu") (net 3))
 (segment (start 83.895 33.655) (end 93.0525 33.655) (width 0.2) (layer "F.Cu") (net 3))
 (segment (start 97.8127 37.0931) (end 97.073 37.8328) (width 0.2) (layer "F.Cu") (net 3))
 (segment (start 97.073 37.8328) (end 98.0198 36.886) (width 0.2) (layer "F.Cu") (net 3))
 (via (at 97.073 37.8328) (size 0.6) (drill 0.3) (layers "F.Cu" "B.Cu") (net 3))
 (via (at 93.98 34.5825) (size 0.6) (drill 0.3) (layers "F.Cu" "B.Cu") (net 3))
 (segment (start 97.8127 37.0931) (end 97.073 37.8328) (width 0.2) (layer "B.Cu") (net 3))
 (segment (start 97.073 37.8328) (end 97.8127 37.0931) (width 0.2) (layer "B.Cu") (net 3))
 (segment (start 97.073 37.6755) (end 97.073 37.8328) (width 0.2) (layer "B.Cu") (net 3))
 (segment (start 93.98 34.5825) (end 97.073 37.6755) (width 0.2) (layer "B.Cu") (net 3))
 (segment (start 109.22 36.195) (end 107.6075 34.5825) (width 0.2) (layer "F.Cu") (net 4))
 (segment (start 86.435 34.925) (end 87.015 35.505) (width 0.2) (layer "F.Cu") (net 4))
 (segment (start 100.6775 35.505) (end 101.6 34.5825) (width 0.2) (layer "F.Cu") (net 4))
 (segment (start 87.015 35.505) (end 100.6775 35.505) (width 0.2) (layer "F.Cu") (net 4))
 (segment (start 107.6075 34.5825) (end 101.6 34.5825) (width 0.2) (layer "F.Cu") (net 4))
 (via (at 101.6 34.5825) (size 0.6) (drill 0.3) (layers "F.Cu" "B.Cu") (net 4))
 (segment (start 92.3675 36.195) (end 83.895 36.195) (width 0.2) (layer "F.Cu") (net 5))
 (segment (start 111.76 35.1528) (end 109.6335 37.2793) (width 0.2) (layer "F.Cu") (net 5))
 (segment (start 104.5151 36.4843) (end 95.3032 36.4843) (width 0.2) (layer "F.Cu") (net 5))
 (segment (start 109.6335 37.2793) (end 105.3101 37.2793) (width 0.2) (layer "F.Cu") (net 5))
 (segment (start 105.3101 37.2793) (end 104.5151 36.4843) (width 0.2) (layer "F.Cu") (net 5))
 (segment (start 95.3032 36.4843) (end 93.98 37.8075) (width 0.2) (layer "F.Cu") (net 5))
 (segment (start 93.98 37.8075) (end 92.3675 36.195) (width 0.2) (layer "F.Cu") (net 5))
 (segment (start 111.76 34.925) (end 111.76 35.1528) (width 0.2) (layer "F.Cu") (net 5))
 (via (at 93.98 37.8075) (size 0.6) (drill 0.3) (layers "F.Cu" "B.Cu") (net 5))
 (segment (start 100.6279 38.7796) (end 87.7496 38.7796) (width 0.2) (layer "F.Cu") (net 6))
 (segment (start 98.3884 33.5356) (end 109.1006 33.5356) (width 0.2) (layer "F.Cu") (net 6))
 (segment (start 109.1006 33.5356) (end 109.22 33.655) (width 0.2) (layer "F.Cu") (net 6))
 (segment (start 98.4259 33.5356) (end 98.3884 33.5356) (width 0.2) (layer "F.Cu") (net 6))
 (segment (start 98.3884 33.5356) (end 98.4259 33.5356) (width 0.2) (layer "F.Cu") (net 6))
 (segment (start 87.7496 38.7796) (end 86.435 37.465) (width 0.2) (layer "F.Cu") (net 6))
 (segment (start 101.6 37.8075) (end 100.6279 38.7796) (width 0.2) (layer "F.Cu") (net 6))
 (via (at 101.6 37.8075) (size 0.6) (drill 0.3) (layers "F.Cu" "B.Cu") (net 6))
 (via (at 98.3884 33.5356) (size 0.6) (drill 0.3) (layers "F.Cu" "B.Cu") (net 6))
 (segment (start 101.6 37.8075) (end 101.6 36.7472) (width 0.2) (layer "B.Cu") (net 6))
 (segment (start 98.4259 33.5356) (end 98.3884 33.5356) (width 0.2) (layer "B.Cu") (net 6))
 (segment (start 98.3884 33.5356) (end 98.4259 33.5356) (width 0.2) (layer "B.Cu") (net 6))
 (segment (start 101.6 36.7472) (end 98.3884 33.5356) (width 0.2) (layer "B.Cu") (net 6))
 (segment (start 98.1656 34.3392) (end 98.5071 34.6807) (width 0.2) (layer "F.Cu") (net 7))
 (segment (start 98.5071 34.6807) (end 97.7786 33.9522) (width 0.2) (layer "F.Cu") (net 7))
 (segment (start 89.069 44.1575) (end 83.895 38.9835) (width 0.2) (layer "F.Cu") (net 7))
 (segment (start 97.7786 33.9522) (end 97.7786 33.2238) (width 0.2) (layer "F.Cu") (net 7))
 (segment (start 97.7786 33.2238) (end 98.6174 32.385) (width 0.2) (layer "F.Cu") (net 7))
 (segment (start 83.895 38.9835) (end 83.895 38.735) (width 0.2) (layer "F.Cu") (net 7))
 (segment (start 98.5071 34.6807) (end 98.1656 34.3392) (width 0.2) (layer "F.Cu") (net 7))
 (segment (start 93.98 44.1575) (end 89.069 44.1575) (width 0.2) (layer "F.Cu") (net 7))
 (segment (start 98.6174 32.385) (end 111.76 32.385) (width 0.2) (layer "F.Cu") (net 7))
 (via (at 93.98 44.1575) (size 0.6) (drill 0.3) (layers "F.Cu" "B.Cu") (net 7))
 (via (at 98.5071 34.6807) (size 0.6) (drill 0.3) (layers "F.Cu" "B.Cu") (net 7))
 (segment (start 93.98 44.1575) (end 98.5071 39.6304) (width 0.2) (layer "B.Cu") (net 7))
 (segment (start 98.5071 34.6807) (end 98.1656 34.3392) (width 0.2) (layer "B.Cu") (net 7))
 (segment (start 98.5071 39.6304) (end 98.5071 34.6807) (width 0.2) (layer "B.Cu") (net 7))
 (segment (start 98.1656 34.3392) (end 98.5071 34.6807) (width 0.2) (layer "B.Cu") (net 7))
 (segment (start 101.6 44.1575) (end 99.5858 42.1433) (width 0.2) (layer "F.Cu") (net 8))
 (segment (start 88.5733 42.1433) (end 86.435 40.005) (width 0.2) (layer "F.Cu") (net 8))
 (segment (start 99.5858 42.1433) (end 88.5733 42.1433) (width 0.2) (layer "F.Cu") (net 8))
 (via (at 101.6 44.1575) (size 0.6) (drill 0.3) (layers "F.Cu" "B.Cu") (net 8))
 (segment (start 109.22 31.4031) (end 111.4719 33.655) (width 0.2) (layer "B.Cu") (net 8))
 (segment (start 112.8453 40.8789) (end 109.5667 44.1575) (width 0.2) (layer "B.Cu") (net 8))
 (segment (start 109.22 31.115) (end 109.22 31.4031) (width 0.2) (layer "B.Cu") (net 8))
 (segment (start 109.5667 44.1575) (end 101.6 44.1575) (width 0.2) (layer "B.Cu") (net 8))
 (segment (start 111.9842 33.655) (end 112.8453 34.5161) (width 0.2) (layer "B.Cu") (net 8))
 (segment (start 112.8453 34.5161) (end 112.8453 40.8789) (width 0.2) (layer "B.Cu") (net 8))
 (segment (start 111.4719 33.655) (end 111.9842 33.655) (width 0.2) (layer "B.Cu") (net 8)))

